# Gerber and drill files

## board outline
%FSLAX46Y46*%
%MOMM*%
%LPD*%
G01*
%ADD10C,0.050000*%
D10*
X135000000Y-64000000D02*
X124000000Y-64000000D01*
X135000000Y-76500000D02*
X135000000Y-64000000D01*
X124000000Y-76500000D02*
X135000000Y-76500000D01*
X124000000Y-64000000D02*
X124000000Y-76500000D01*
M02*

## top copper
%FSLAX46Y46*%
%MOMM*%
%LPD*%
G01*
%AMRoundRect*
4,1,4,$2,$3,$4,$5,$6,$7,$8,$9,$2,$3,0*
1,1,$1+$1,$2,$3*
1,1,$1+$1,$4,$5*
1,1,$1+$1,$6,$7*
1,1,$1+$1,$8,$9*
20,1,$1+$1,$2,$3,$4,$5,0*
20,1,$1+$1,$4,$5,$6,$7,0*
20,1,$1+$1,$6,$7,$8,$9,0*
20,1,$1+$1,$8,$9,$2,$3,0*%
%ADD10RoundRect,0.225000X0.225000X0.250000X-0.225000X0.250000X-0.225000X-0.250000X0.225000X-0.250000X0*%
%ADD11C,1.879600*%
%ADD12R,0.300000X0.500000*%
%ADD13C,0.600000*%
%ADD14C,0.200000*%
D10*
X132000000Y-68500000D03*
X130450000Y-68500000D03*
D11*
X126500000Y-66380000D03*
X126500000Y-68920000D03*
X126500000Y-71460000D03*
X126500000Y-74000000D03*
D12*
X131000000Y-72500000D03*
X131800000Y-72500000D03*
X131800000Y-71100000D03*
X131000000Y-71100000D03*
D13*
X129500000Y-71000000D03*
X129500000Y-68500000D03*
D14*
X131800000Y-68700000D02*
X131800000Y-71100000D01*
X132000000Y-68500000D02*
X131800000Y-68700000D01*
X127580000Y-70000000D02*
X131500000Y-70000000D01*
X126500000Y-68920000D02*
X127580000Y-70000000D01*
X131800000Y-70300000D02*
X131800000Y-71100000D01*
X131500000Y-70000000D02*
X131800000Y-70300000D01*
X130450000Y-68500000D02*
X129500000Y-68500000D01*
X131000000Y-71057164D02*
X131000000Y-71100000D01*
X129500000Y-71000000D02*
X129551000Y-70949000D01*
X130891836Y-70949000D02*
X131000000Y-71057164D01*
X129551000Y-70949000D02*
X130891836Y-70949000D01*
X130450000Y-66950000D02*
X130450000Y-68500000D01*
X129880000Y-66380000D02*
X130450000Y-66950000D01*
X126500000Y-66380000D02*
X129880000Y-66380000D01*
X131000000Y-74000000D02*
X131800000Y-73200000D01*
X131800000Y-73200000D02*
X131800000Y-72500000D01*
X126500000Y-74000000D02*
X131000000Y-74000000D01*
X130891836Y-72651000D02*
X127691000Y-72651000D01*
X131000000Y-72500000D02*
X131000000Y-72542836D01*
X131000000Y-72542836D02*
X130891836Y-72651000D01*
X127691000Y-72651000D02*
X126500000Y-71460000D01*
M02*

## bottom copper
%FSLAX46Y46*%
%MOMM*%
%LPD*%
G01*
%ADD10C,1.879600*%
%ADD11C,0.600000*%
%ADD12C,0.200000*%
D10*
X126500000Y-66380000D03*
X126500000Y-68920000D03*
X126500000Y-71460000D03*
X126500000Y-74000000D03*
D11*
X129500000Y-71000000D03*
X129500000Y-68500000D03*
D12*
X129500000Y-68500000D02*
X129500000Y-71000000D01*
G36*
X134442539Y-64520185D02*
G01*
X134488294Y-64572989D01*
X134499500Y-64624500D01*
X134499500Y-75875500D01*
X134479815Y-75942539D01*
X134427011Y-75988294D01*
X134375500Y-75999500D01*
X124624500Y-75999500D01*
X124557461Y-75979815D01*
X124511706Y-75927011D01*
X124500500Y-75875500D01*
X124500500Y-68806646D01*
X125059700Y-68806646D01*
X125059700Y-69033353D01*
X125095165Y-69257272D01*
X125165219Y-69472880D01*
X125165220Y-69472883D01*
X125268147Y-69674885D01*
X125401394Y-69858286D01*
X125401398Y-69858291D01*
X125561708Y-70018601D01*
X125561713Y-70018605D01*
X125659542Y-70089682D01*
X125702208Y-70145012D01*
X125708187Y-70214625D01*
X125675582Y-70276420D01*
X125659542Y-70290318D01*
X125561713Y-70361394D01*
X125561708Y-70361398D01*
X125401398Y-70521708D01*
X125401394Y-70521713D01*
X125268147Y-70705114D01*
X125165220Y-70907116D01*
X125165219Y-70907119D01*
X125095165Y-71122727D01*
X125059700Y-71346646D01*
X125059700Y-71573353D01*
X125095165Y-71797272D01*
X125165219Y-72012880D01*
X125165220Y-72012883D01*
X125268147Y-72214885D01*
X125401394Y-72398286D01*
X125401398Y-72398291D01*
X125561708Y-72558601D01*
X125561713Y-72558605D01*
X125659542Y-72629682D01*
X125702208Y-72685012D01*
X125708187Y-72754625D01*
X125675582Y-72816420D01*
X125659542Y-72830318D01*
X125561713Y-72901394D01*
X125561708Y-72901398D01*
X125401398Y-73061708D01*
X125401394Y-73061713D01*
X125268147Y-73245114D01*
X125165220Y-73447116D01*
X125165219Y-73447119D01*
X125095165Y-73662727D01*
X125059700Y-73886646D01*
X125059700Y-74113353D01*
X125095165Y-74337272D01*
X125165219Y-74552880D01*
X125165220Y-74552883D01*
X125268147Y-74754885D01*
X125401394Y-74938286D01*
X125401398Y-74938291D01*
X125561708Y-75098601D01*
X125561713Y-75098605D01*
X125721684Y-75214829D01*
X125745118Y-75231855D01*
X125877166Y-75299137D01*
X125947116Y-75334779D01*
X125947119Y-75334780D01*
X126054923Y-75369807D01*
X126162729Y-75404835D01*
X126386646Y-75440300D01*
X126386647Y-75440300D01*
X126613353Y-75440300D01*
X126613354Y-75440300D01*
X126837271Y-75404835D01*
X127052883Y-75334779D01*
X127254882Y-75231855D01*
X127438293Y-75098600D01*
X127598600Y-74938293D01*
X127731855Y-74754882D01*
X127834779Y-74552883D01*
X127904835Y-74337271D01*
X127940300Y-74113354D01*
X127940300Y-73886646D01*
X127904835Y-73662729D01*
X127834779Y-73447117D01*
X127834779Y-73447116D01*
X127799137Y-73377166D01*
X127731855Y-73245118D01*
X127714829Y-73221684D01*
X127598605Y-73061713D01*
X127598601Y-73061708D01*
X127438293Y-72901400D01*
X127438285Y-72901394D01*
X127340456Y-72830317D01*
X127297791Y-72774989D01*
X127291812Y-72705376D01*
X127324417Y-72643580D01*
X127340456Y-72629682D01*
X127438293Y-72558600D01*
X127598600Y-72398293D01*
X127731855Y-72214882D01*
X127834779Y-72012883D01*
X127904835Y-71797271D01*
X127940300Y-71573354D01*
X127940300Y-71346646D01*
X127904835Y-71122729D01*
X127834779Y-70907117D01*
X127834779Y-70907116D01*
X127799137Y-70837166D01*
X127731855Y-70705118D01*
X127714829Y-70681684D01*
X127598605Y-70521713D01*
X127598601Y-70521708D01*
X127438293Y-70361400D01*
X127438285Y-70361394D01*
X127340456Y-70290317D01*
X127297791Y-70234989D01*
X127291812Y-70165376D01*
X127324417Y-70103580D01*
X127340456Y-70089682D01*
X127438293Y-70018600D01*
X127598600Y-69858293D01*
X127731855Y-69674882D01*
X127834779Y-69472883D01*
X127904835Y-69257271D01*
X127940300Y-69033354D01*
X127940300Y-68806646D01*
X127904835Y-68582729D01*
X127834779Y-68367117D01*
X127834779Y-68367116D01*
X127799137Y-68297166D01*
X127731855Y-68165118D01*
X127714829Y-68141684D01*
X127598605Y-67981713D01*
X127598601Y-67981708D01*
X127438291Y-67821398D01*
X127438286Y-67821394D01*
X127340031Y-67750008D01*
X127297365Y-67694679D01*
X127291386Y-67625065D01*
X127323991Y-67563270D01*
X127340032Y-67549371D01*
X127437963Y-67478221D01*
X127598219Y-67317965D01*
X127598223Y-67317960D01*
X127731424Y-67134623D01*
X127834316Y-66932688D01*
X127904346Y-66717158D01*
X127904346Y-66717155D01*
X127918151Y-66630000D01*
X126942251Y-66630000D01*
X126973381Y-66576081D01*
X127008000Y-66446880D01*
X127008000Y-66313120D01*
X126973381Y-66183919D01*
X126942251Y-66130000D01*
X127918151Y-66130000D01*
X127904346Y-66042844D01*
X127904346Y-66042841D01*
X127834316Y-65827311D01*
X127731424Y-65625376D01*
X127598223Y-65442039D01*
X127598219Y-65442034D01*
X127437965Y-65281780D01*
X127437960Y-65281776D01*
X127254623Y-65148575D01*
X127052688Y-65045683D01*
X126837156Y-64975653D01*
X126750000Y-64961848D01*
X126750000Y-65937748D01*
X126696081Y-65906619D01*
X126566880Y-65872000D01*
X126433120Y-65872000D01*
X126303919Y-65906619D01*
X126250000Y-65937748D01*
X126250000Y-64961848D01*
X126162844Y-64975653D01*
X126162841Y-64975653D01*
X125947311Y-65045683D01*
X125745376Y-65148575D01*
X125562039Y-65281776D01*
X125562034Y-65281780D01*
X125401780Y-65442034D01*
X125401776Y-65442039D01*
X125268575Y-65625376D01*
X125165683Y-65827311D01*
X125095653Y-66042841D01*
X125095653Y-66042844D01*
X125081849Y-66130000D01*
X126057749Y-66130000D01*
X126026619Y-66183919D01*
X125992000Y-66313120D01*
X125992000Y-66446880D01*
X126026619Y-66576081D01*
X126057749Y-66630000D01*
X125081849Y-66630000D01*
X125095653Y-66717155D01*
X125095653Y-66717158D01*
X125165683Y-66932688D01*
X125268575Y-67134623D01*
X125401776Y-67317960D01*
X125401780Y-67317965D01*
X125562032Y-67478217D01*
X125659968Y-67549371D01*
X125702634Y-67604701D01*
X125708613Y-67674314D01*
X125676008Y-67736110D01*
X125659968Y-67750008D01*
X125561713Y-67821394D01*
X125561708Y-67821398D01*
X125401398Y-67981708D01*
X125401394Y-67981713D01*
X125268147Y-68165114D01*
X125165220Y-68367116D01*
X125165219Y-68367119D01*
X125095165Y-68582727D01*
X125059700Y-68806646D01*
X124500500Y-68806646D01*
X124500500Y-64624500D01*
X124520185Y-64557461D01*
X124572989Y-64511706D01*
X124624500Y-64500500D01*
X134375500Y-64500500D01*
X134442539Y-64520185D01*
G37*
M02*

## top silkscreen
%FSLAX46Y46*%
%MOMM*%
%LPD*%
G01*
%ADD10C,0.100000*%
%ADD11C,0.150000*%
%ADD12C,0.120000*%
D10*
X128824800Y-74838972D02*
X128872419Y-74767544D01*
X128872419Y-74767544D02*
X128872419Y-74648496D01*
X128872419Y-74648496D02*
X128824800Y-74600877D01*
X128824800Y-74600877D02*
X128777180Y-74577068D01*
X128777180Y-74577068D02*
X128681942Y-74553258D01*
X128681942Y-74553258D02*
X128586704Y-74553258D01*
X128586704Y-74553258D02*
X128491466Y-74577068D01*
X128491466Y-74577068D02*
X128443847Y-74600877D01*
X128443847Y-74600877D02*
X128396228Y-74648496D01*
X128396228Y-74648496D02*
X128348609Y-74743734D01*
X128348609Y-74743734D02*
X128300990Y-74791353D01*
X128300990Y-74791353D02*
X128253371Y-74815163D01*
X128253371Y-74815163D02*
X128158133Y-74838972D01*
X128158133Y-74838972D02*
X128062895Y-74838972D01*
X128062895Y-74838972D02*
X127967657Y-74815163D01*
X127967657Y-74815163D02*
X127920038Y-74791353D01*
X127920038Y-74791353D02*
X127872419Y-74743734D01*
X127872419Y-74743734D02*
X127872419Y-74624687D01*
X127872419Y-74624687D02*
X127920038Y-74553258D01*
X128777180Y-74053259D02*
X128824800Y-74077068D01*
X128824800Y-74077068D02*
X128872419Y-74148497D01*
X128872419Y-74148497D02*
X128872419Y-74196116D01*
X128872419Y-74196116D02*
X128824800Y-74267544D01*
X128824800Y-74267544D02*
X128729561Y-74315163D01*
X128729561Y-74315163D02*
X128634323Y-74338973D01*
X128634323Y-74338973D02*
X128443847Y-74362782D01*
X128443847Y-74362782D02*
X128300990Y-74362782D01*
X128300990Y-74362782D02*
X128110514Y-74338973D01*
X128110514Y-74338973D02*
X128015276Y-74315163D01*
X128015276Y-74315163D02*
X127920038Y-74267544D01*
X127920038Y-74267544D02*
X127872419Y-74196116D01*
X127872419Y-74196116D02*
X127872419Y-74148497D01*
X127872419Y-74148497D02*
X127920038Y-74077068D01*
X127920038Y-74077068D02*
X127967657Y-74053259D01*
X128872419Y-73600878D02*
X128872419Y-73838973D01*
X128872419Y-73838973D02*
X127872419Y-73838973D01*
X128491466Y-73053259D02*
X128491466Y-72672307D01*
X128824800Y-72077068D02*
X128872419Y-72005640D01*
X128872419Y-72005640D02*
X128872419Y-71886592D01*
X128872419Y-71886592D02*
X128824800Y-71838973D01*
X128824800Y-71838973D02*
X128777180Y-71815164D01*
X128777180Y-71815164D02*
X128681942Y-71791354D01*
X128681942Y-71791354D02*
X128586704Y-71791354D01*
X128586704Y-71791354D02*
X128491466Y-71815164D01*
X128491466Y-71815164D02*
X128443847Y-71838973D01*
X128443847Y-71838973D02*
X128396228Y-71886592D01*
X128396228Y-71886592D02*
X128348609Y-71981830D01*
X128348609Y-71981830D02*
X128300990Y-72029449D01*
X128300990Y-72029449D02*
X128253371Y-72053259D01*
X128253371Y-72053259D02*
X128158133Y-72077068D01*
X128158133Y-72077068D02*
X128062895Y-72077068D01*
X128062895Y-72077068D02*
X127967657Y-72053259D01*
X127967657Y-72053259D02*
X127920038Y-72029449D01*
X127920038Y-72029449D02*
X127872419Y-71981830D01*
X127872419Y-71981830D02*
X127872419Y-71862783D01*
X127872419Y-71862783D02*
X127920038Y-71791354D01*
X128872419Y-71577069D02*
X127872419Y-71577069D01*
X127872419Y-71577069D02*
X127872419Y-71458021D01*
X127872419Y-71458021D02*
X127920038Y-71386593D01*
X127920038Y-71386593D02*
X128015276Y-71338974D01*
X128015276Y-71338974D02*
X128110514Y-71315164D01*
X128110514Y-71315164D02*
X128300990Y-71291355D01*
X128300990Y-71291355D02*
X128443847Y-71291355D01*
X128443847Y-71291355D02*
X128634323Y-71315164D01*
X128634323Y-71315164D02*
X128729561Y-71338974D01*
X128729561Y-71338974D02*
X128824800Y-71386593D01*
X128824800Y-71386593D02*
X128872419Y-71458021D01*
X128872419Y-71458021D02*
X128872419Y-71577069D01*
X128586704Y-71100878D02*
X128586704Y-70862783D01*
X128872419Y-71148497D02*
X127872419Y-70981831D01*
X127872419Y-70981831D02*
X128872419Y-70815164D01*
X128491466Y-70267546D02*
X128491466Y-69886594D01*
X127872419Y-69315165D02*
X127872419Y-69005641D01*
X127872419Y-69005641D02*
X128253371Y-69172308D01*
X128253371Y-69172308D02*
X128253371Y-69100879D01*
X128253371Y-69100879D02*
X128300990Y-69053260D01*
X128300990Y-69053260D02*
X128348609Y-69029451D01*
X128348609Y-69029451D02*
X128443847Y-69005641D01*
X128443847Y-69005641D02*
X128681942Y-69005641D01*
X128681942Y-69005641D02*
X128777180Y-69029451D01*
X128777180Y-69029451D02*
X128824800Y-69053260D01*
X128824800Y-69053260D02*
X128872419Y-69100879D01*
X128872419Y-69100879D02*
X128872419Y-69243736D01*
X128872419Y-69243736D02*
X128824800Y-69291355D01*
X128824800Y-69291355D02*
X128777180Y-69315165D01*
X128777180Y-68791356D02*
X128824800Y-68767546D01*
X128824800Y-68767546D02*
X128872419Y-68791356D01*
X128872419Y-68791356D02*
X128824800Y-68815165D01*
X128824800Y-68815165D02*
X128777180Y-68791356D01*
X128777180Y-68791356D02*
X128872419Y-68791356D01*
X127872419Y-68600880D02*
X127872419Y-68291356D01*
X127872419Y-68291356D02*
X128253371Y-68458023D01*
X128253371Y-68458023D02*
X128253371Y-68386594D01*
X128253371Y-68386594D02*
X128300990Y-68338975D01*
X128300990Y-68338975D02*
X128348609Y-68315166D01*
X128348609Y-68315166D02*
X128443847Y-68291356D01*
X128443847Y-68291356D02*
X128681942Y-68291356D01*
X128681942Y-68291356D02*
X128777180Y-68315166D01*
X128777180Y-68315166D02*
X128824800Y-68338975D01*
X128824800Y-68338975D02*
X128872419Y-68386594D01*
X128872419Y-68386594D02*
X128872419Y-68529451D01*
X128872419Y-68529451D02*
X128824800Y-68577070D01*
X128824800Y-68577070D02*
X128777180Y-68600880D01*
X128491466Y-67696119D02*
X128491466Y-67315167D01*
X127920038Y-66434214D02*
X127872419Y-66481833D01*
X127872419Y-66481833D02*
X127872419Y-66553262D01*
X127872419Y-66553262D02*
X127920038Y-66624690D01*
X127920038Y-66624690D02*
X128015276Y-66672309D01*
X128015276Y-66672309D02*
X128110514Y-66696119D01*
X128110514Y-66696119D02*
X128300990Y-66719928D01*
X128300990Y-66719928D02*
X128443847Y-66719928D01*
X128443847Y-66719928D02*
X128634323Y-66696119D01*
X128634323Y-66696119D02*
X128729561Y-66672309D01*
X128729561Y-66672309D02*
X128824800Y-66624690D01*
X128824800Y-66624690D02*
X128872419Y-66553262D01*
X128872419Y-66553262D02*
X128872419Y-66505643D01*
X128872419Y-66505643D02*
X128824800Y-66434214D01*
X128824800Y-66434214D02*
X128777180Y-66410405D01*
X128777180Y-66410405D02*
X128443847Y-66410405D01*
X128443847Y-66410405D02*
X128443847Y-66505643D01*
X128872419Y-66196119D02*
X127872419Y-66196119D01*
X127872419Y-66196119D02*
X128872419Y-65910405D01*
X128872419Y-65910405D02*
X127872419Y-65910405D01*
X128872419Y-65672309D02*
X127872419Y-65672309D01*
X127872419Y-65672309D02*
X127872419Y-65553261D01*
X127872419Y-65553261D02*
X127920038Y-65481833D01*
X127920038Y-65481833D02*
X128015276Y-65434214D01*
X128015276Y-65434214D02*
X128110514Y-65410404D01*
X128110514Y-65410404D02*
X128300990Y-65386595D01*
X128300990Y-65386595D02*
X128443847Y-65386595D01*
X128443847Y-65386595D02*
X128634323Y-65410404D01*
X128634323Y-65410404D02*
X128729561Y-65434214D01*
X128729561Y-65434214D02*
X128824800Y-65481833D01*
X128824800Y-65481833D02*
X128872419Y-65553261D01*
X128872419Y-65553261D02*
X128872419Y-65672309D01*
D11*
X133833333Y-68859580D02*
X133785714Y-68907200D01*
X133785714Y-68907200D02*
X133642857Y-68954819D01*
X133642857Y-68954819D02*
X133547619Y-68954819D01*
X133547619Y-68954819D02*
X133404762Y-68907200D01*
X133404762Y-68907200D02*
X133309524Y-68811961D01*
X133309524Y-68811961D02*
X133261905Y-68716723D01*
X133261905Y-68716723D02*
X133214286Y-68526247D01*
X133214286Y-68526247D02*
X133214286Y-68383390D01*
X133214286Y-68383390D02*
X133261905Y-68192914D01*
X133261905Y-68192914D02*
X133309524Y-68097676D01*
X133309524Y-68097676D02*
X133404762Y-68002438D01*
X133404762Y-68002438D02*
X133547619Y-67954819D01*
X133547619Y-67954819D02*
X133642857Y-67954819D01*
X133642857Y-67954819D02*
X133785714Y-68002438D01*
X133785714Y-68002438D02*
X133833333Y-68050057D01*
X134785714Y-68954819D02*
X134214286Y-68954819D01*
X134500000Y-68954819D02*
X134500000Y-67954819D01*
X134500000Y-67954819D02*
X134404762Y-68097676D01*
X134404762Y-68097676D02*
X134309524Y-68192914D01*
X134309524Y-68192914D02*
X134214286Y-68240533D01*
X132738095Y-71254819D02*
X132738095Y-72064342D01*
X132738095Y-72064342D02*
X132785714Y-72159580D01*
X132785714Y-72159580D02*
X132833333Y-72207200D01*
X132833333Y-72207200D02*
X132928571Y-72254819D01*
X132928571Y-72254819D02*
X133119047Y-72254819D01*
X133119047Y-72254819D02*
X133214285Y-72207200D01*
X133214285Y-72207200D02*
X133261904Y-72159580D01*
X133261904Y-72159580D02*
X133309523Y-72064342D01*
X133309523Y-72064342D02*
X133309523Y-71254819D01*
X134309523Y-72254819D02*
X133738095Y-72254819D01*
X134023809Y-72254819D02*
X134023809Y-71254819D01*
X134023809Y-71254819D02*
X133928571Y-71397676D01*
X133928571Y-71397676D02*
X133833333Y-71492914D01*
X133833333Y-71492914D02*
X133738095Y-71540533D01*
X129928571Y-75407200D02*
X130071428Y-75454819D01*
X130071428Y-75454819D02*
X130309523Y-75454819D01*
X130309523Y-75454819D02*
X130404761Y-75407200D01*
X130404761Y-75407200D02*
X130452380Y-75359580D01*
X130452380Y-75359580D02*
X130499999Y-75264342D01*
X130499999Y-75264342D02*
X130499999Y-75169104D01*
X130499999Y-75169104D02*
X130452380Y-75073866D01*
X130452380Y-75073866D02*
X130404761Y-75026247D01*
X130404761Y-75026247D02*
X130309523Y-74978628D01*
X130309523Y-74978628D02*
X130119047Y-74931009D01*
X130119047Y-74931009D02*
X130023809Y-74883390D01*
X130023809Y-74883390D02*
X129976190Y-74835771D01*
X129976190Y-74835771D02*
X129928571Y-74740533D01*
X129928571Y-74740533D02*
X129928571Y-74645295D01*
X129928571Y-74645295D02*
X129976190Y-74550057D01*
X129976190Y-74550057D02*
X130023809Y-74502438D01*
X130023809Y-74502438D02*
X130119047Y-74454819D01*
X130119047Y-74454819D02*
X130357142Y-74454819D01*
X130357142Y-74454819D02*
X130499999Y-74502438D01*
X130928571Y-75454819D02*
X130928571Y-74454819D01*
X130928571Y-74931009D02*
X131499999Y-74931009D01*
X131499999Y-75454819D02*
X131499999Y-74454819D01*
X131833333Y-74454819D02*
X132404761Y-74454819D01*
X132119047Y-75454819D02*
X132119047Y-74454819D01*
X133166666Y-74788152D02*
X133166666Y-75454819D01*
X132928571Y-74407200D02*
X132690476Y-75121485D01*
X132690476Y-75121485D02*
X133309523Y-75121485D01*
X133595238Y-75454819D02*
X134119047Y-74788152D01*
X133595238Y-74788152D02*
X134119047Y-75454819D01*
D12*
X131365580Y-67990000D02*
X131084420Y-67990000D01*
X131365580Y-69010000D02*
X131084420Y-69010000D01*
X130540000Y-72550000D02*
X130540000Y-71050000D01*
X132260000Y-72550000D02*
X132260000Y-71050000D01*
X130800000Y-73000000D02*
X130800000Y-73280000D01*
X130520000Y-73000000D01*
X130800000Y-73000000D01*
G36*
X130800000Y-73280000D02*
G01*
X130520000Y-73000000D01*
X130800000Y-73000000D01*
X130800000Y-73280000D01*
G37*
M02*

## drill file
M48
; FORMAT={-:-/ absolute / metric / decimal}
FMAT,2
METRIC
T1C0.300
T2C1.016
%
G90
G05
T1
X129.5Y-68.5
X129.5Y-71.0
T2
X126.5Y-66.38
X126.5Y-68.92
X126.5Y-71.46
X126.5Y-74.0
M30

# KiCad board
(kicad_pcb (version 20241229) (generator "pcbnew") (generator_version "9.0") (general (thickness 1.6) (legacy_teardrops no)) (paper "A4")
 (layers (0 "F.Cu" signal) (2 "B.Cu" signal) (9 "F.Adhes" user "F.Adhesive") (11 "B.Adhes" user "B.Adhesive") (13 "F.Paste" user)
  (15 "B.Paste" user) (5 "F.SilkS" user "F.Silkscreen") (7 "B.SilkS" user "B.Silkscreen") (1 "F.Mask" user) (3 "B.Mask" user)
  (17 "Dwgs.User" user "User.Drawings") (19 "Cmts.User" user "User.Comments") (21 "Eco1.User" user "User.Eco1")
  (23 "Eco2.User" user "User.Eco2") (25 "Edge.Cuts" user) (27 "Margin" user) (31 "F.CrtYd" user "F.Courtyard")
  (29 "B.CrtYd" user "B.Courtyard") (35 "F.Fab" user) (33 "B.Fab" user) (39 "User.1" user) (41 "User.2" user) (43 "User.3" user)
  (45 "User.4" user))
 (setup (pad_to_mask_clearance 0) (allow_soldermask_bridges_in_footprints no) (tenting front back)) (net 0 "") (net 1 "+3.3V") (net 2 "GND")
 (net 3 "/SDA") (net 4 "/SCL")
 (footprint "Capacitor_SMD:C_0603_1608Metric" (layer "F.Cu") (at 131.225 68.5 180)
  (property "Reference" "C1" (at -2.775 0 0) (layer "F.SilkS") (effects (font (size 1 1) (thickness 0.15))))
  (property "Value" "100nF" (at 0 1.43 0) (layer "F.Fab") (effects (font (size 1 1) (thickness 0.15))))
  (fp_line (start -0.14058 0.51) (end 0.14058 0.51) (stroke (width 0.12) (type solid)) (layer "F.SilkS"))
  (fp_line (start -0.14058 -0.51) (end 0.14058 -0.51) (stroke (width 0.12) (type solid)) (layer "F.SilkS"))
  (pad "1" smd roundrect (at -0.775 0 180) (size 0.9 0.95) (layers "F.Cu" "F.Mask" "F.Paste") (roundrect_rratio 0.25) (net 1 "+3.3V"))
  (pad "2" smd roundrect (at 0.775 0 180) (size 0.9 0.95) (layers "F.Cu" "F.Mask" "F.Paste") (roundrect_rratio 0.25) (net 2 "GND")))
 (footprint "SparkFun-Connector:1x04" (layer "F.Cu") (at 126.5 66.38 -90)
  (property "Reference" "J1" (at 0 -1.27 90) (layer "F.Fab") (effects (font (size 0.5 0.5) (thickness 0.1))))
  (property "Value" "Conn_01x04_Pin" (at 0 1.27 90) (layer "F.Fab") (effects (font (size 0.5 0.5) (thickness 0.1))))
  (pad "1" thru_hole circle (at 0 0) (size 1.8796 1.8796) (drill 1.016) (layers "*.Cu" "*.Mask") (remove_unused_layers yes)
   (keep_end_layers yes) (zone_layer_connections) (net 2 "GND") (thermal_bridge_angle 0))
  (pad "2" thru_hole circle (at 2.54 0) (size 1.8796 1.8796) (drill 1.016) (layers "*.Cu" "*.Mask") (remove_unused_layers yes)
   (keep_end_layers yes) (zone_layer_connections) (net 1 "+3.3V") (thermal_bridge_angle 0))
  (pad "3" thru_hole circle (at 5.08 0) (size 1.8796 1.8796) (drill 1.016) (layers "*.Cu" "*.Mask") (remove_unused_layers yes)
   (keep_end_layers yes) (zone_layer_connections) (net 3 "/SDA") (thermal_bridge_angle 0))
  (pad "4" thru_hole circle (at 7.62 0) (size 1.8796 1.8796) (drill 1.016) (layers "*.Cu" "*.Mask") (remove_unused_layers yes)
   (keep_end_layers yes) (zone_layer_connections) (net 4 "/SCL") (thermal_bridge_angle 0)))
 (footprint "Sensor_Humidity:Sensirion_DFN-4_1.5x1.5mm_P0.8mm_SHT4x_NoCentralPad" (layer "F.Cu") (at 131.4 71.8 90)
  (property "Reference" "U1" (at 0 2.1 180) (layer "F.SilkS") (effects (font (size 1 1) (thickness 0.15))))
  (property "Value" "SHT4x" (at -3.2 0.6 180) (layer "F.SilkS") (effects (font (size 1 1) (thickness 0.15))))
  (fp_line (start -0.75 -0.86) (end 0.75 -0.86) (stroke (width 0.12) (type solid)) (layer "F.SilkS"))
  (fp_line (start -0.75 0.86) (end 0.75 0.86) (stroke (width 0.12) (type solid)) (layer "F.SilkS"))
  (fp_poly
   (pts (xy -1.2 -0.6) (xy -1.48 -0.6) (xy -1.2 -0.88) (xy -1.2 -0.6)) (stroke (width 0.12) (type solid)) (fill yes) (layer "F.SilkS"))
  (pad "1" smd rect (at -0.7 -0.4 90) (size 0.5 0.3) (layers "F.Cu" "F.Mask" "F.Paste") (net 3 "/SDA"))
  (pad "2" smd rect (at -0.7 0.4 90) (size 0.5 0.3) (layers "F.Cu" "F.Mask" "F.Paste") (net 4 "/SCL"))
  (pad "3" smd rect (at 0.7 0.4 90) (size 0.5 0.3) (layers "F.Cu" "F.Mask" "F.Paste") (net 1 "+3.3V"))
  (pad "4" smd rect (at 0.7 -0.4 90) (size 0.5 0.3) (layers "F.Cu" "F.Mask" "F.Paste") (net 2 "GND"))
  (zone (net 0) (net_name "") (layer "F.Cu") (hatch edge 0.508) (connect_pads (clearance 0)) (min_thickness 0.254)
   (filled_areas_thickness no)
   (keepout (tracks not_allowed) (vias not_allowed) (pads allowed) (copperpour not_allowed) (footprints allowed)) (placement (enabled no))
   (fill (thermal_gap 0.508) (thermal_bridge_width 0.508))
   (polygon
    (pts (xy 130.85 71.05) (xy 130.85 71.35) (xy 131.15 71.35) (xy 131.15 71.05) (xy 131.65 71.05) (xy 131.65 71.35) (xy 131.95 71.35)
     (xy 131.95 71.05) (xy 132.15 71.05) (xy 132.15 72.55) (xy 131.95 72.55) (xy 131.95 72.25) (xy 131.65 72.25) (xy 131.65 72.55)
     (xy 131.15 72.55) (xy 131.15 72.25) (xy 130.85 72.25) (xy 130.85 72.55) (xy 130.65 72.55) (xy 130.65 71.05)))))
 (gr_line (start 135 64) (end 124 64) (stroke (width 0.05) (type default)) (layer "Edge.Cuts"))
 (gr_line (start 135 76.5) (end 135 64) (stroke (width 0.05) (type default)) (layer "Edge.Cuts"))
 (gr_line (start 124 76.5) (end 135 76.5) (stroke (width 0.05) (type default)) (layer "Edge.Cuts"))
 (gr_line (start 124 64) (end 124 76.5) (stroke (width 0.05) (type default)) (layer "Edge.Cuts"))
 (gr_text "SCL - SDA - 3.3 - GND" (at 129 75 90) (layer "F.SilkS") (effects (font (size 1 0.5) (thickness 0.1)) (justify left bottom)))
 (segment (start 131.8 68.7) (end 131.8 71.1) (width 0.2) (layer "F.Cu") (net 1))
 (segment (start 132 68.5) (end 131.8 68.7) (width 0.2) (layer "F.Cu") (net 1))
 (segment (start 127.58 70) (end 131.5 70) (width 0.2) (layer "F.Cu") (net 1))
 (segment (start 126.5 68.92) (end 127.58 70) (width 0.2) (layer "F.Cu") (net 1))
 (segment (start 131.8 70.3) (end 131.8 71.1) (width 0.2) (layer "F.Cu") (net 1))
 (segment (start 131.5 70) (end 131.8 70.3) (width 0.2) (layer "F.Cu") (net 1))
 (segment (start 130.45 68.5) (end 129.5 68.5) (width 0.2) (layer "F.Cu") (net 2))
 (segment (start 131 71.057164) (end 131 71.1) (width 0.2) (layer "F.Cu") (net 2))
 (segment (start 129.5 71) (end 129.551 70.949) (width 0.2) (layer "F.Cu") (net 2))
 (segment (start 130.891836 70.949) (end 131 71.057164) (width 0.2) (layer "F.Cu") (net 2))
 (segment (start 129.551 70.949) (end 130.891836 70.949) (width 0.2) (layer "F.Cu") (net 2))
 (segment (start 130.45 66.95) (end 130.45 68.5) (width 0.2) (layer "F.Cu") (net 2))
 (segment (start 129.88 66.38) (end 130.45 66.95) (width 0.2) (layer "F.Cu") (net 2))
 (segment (start 126.5 66.38) (end 129.88 66.38) (width 0.2) (layer "F.Cu") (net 2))
 (via (at 129.5 71) (size 0.6) (drill 0.3) (layers "F.Cu" "B.Cu") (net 2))
 (via (at 129.5 68.5) (size 0.6) (drill 0.3) (layers "F.Cu" "B.Cu") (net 2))
 (segment (start 129.5 68.5) (end 129.5 71) (width 0.2) (layer "B.Cu") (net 2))
 (segment (start 131 74) (end 131.8 73.2) (width 0.2) (layer "F.Cu") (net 4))
 (segment (start 131.8 73.2) (end 131.8 72.5) (width 0.2) (layer "F.Cu") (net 4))
 (segment (start 126.5 74) (end 131 74) (width 0.2) (layer "F.Cu") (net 4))
 (segment (start 130.891836 72.651) (end 127.691 72.651) (width 0.2) (layer "F.Cu") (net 3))
 (segment (start 131 72.5) (end 131 72.542836) (width 0.2) (layer "F.Cu") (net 3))
 (segment (start 131 72.542836) (end 130.891836 72.651) (width 0.2) (layer "F.Cu") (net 3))
 (segment (start 127.691 72.651) (end 126.5 71.46) (width 0.2) (layer "F.Cu") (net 3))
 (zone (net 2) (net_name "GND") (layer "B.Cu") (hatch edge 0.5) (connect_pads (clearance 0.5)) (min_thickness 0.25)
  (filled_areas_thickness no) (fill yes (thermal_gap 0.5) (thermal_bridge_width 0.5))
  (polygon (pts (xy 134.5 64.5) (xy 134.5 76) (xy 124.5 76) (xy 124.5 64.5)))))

